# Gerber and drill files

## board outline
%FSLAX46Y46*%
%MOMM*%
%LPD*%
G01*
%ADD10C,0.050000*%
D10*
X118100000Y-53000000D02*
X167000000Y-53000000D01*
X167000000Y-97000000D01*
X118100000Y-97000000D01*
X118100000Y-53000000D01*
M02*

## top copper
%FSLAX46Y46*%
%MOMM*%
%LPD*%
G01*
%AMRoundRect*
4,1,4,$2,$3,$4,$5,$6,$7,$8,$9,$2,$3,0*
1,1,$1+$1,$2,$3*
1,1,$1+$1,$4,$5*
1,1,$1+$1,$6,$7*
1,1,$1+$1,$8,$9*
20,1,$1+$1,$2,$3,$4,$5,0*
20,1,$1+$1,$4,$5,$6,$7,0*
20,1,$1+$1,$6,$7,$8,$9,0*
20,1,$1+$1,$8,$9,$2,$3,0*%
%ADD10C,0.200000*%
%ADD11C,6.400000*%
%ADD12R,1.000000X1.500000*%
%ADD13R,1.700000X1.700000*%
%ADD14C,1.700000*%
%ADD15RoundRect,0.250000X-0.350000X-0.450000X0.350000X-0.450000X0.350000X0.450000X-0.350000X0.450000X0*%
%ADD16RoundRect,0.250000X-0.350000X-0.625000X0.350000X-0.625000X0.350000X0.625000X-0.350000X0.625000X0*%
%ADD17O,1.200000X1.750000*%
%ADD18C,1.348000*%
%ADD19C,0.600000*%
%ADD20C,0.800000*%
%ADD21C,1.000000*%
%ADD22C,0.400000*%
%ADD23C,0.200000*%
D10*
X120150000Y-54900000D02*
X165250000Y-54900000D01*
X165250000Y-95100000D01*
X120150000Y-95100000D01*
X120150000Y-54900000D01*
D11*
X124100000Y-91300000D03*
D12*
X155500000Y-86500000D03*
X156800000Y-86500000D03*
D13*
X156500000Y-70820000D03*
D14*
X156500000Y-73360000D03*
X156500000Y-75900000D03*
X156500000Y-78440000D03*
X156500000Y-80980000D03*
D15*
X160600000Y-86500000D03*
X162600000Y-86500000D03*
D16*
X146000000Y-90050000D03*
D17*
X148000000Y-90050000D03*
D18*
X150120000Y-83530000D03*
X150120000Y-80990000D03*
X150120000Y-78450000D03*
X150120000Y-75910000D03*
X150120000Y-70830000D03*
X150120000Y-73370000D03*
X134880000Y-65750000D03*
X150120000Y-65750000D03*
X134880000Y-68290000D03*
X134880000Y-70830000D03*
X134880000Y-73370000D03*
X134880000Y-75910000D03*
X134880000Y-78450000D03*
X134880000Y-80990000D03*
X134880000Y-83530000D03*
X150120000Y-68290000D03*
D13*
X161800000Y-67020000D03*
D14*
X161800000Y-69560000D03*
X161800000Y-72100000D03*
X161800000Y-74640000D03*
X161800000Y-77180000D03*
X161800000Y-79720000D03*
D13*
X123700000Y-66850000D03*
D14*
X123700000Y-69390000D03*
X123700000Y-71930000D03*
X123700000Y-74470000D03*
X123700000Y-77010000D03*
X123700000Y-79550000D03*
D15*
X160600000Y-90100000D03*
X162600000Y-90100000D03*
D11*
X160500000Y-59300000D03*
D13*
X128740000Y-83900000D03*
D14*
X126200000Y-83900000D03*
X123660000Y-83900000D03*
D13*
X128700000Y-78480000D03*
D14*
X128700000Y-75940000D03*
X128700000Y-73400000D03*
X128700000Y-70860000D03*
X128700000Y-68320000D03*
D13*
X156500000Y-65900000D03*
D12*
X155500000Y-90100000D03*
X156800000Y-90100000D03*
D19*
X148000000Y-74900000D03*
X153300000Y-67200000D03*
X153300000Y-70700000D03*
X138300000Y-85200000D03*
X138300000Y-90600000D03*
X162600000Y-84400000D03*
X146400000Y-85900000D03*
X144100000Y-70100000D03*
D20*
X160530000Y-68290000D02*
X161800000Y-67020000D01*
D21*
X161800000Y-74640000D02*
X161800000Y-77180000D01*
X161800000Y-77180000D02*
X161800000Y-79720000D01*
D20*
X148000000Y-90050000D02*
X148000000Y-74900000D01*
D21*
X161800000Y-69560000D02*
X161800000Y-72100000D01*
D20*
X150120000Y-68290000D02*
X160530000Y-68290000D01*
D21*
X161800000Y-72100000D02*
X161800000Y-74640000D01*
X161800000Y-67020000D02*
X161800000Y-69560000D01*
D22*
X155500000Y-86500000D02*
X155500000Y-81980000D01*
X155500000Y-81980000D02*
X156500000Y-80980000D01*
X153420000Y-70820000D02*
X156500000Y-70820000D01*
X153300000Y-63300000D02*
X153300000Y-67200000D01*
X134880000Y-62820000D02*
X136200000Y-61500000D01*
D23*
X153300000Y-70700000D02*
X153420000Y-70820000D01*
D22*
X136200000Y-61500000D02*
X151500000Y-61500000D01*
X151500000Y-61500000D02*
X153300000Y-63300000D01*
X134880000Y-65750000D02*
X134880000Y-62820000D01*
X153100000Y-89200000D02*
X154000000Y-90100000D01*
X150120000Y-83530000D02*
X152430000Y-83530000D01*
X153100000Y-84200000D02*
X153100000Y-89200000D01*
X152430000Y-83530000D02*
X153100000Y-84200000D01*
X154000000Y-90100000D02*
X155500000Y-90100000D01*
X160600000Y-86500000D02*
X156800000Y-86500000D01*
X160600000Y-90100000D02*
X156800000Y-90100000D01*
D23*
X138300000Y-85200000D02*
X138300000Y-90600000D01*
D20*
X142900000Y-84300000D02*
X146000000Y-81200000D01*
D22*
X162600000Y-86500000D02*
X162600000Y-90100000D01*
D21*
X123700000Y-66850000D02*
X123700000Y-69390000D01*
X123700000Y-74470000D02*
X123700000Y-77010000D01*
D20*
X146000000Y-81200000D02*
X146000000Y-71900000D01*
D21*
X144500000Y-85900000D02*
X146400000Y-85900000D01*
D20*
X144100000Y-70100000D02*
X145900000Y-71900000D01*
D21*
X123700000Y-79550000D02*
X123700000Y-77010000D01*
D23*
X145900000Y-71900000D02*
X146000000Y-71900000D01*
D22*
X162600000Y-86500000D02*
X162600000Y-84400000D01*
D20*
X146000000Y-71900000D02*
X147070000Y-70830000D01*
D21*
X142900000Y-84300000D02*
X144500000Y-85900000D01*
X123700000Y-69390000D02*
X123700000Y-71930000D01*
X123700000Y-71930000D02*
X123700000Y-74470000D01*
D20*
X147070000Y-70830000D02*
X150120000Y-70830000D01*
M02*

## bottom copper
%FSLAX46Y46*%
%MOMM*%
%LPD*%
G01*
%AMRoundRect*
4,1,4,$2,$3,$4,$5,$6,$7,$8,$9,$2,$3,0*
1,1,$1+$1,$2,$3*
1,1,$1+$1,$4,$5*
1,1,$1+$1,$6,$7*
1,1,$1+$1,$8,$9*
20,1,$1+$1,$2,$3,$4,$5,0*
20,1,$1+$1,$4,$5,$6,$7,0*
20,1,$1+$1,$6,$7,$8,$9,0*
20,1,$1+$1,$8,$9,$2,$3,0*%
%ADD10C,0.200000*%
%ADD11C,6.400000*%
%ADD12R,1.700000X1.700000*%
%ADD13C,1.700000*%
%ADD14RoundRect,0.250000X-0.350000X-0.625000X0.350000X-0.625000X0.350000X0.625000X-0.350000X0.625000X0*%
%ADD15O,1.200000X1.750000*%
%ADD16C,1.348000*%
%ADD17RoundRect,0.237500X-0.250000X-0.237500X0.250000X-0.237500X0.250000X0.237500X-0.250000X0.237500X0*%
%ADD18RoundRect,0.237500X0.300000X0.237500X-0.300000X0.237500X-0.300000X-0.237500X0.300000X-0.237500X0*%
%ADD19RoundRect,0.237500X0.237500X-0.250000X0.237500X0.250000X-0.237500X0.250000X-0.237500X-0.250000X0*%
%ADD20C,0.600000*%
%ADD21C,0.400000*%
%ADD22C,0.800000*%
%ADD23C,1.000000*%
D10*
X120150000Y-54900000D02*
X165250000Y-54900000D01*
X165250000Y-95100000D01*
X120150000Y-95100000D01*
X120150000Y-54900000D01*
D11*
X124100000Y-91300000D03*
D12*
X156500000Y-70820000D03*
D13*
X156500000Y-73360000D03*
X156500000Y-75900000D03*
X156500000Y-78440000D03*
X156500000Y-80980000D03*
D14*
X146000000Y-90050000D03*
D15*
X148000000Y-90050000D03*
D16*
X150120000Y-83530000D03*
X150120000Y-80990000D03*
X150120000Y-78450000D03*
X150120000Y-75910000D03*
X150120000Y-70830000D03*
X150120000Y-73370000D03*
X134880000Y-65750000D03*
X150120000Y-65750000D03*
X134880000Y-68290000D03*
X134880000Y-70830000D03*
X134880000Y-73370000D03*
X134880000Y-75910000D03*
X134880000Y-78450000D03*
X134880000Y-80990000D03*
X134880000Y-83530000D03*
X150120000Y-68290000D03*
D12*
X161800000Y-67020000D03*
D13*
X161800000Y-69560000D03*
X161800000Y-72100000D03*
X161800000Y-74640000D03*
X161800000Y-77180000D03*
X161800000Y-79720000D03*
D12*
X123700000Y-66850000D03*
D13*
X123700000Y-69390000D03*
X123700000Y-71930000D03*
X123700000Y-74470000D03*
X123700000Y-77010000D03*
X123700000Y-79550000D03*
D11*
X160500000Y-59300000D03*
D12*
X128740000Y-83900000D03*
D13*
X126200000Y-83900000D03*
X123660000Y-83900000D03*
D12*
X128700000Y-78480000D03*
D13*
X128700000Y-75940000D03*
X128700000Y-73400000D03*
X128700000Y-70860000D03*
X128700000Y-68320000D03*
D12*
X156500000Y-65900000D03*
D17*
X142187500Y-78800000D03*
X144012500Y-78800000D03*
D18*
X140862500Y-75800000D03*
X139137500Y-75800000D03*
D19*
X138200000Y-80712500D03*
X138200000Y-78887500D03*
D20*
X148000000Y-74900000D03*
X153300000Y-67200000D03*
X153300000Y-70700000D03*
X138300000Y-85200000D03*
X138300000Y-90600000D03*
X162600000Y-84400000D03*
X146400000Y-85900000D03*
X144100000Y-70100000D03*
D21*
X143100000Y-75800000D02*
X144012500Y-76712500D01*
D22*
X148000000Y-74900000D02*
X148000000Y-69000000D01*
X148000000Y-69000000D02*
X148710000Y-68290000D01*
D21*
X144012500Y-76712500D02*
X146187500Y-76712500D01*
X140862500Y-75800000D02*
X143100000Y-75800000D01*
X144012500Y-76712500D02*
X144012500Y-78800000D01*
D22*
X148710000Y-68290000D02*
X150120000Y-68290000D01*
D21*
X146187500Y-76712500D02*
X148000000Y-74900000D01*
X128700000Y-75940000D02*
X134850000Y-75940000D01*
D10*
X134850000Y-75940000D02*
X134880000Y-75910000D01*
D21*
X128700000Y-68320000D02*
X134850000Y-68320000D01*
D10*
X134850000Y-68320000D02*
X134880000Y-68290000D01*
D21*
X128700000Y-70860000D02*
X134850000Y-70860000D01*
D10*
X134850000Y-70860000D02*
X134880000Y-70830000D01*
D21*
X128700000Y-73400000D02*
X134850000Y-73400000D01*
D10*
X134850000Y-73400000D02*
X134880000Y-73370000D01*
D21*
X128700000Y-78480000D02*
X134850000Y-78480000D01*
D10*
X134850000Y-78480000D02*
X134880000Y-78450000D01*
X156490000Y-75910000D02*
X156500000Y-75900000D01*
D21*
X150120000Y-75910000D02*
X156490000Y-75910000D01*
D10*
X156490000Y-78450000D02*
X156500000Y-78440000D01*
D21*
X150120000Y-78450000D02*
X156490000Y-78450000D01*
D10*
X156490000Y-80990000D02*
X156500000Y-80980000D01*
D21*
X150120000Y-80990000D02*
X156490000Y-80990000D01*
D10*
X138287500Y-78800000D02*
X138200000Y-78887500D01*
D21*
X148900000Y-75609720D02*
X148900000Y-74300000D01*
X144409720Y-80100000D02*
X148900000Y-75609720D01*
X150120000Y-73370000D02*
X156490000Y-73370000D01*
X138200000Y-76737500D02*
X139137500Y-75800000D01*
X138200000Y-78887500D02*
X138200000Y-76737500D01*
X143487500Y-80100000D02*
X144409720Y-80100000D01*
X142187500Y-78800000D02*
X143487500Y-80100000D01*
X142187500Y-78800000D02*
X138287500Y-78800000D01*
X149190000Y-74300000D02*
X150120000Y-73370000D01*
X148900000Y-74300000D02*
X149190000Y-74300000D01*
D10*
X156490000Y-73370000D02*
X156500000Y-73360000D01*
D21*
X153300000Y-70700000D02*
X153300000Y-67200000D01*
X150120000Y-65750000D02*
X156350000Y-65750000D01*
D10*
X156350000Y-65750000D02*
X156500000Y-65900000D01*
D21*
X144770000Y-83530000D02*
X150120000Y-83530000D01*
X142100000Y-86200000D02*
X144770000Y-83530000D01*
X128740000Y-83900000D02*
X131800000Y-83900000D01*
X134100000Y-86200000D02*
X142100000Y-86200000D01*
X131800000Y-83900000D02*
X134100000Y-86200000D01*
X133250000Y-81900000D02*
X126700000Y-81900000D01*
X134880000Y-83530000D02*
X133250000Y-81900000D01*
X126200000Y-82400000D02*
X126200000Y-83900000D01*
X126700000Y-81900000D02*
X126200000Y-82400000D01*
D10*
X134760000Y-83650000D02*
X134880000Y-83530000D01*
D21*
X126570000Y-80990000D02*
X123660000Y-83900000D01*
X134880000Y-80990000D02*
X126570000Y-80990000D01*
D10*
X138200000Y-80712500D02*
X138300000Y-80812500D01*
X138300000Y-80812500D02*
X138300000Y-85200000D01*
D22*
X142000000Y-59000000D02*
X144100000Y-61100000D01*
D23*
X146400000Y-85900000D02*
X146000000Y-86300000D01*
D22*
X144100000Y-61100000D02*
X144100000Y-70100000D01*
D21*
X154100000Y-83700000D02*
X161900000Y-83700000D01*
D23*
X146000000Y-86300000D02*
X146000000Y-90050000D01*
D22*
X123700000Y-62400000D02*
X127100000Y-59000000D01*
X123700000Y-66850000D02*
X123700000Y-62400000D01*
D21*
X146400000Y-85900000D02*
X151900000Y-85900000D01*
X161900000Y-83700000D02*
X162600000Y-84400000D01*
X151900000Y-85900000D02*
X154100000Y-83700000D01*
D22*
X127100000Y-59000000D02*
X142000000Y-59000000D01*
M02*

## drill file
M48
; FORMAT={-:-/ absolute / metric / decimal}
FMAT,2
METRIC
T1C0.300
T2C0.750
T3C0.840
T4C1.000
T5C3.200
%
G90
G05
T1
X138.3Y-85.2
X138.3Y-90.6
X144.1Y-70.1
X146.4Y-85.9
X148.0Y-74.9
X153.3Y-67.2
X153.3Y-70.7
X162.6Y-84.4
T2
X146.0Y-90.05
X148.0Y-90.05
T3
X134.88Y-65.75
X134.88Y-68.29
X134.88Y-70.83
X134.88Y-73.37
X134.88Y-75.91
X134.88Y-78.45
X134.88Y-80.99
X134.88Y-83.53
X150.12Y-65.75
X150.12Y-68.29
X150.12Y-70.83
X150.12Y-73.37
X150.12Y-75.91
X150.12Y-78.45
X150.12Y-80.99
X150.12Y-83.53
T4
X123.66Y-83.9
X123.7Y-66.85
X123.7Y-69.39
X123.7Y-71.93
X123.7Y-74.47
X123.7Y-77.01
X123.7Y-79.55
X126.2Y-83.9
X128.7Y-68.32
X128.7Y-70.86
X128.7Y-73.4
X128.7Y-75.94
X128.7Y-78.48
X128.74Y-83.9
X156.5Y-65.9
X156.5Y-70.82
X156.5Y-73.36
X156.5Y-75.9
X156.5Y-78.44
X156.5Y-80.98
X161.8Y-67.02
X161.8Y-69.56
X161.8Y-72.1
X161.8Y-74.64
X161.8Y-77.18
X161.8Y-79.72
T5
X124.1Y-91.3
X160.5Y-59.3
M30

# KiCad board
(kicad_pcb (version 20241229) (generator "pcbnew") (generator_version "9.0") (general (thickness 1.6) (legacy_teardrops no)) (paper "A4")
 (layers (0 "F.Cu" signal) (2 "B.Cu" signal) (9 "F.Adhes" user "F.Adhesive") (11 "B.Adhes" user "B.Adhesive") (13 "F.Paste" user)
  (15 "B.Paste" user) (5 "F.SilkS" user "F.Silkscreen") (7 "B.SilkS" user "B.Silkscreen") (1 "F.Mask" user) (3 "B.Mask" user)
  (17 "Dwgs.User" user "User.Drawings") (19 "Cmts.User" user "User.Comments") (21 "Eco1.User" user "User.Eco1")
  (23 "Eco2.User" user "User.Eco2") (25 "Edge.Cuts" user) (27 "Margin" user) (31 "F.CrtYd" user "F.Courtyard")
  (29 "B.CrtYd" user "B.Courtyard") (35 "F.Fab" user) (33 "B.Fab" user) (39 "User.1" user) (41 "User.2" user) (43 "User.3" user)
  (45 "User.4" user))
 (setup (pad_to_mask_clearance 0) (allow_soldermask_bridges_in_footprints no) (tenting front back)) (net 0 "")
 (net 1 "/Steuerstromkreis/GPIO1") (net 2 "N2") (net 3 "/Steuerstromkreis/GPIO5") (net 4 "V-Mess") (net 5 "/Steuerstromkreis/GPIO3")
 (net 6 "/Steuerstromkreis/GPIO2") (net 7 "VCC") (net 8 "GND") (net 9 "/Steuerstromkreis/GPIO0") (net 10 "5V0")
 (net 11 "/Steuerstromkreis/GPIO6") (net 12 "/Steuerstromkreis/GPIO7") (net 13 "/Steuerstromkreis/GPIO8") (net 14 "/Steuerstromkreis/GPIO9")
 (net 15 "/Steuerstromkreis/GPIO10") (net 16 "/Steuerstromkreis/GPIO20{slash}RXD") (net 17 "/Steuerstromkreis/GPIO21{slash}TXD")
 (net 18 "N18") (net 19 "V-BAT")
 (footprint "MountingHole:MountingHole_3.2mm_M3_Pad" (layer "F.Cu") (at 124.1 91.3)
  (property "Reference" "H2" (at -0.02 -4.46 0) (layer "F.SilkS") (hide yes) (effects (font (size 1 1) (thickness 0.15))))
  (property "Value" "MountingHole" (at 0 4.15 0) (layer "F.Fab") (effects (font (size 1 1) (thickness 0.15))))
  (pad "1" thru_hole circle (at 0 0) (size 6.4 6.4) (drill 3.2) (layers "*.Cu" "*.Mask") (remove_unused_layers no) (zone_connect 2)))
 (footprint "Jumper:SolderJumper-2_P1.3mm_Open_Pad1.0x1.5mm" (layer "F.Cu") (at 156.15 86.5)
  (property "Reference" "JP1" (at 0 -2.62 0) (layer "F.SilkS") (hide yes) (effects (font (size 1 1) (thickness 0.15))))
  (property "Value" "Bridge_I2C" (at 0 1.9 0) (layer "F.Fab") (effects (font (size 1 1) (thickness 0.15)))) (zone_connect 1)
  (pad "1" smd rect (at -0.65 0) (size 1 1.5) (layers "F.Cu" "F.Mask") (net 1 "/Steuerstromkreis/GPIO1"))
  (pad "2" smd rect (at 0.65 0) (size 1 1.5) (layers "F.Cu" "F.Mask") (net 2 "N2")))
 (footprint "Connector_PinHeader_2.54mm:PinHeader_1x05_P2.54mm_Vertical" (layer "F.Cu") (at 156.5 70.82)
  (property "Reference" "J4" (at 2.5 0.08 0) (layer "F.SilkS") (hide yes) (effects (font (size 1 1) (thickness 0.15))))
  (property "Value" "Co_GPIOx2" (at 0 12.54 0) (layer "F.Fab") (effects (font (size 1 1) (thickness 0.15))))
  (pad "1" thru_hole rect (at 0 0) (size 1.7 1.7) (drill 1) (layers "*.Cu" "*.Mask") (remove_unused_layers no)
   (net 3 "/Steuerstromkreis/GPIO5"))
  (pad "2" thru_hole circle (at 0 2.54) (size 1.7 1.7) (drill 1) (layers "*.Cu" "*.Mask") (remove_unused_layers no) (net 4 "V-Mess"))
  (pad "3" thru_hole circle (at 0 5.08) (size 1.7 1.7) (drill 1) (layers "*.Cu" "*.Mask") (remove_unused_layers no)
   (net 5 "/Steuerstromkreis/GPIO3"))
  (pad "4" thru_hole circle (at 0 7.62) (size 1.7 1.7) (drill 1) (layers "*.Cu" "*.Mask") (remove_unused_layers no)
   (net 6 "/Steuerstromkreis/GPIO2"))
  (pad "5" thru_hole circle (at 0 10.16) (size 1.7 1.7) (drill 1) (layers "*.Cu" "*.Mask") (remove_unused_layers no)
   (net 1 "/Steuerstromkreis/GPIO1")))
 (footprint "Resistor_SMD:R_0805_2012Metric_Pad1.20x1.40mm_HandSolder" (layer "F.Cu") (at 161.6 86.5)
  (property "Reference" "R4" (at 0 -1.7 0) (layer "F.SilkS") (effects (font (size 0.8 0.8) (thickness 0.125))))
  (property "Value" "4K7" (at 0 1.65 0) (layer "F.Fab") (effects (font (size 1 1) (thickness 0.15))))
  (pad "1" smd roundrect (at -1 0) (size 1.2 1.4) (layers "F.Cu" "F.Mask" "F.Paste") (roundrect_rratio 0.208333) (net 2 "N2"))
  (pad "2" smd roundrect (at 1 0) (size 1.2 1.4) (layers "F.Cu" "F.Mask" "F.Paste") (roundrect_rratio 0.208333) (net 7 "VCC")))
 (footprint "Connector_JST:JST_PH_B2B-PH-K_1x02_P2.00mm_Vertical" (layer "F.Cu") (at 146 90.05)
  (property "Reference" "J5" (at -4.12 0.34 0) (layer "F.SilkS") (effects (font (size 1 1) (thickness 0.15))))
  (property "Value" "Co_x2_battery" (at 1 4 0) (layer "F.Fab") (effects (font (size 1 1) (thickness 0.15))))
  (pad "1" thru_hole roundrect (at 0 0) (size 1.2 1.75) (drill 0.75) (layers "*.Cu" "*.Mask") (remove_unused_layers no)
   (roundrect_rratio 0.208333) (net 7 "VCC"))
  (pad "2" thru_hole oval (at 2 0) (size 1.2 1.75) (drill 0.75) (layers "*.Cu" "*.Mask") (remove_unused_layers no) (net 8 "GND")))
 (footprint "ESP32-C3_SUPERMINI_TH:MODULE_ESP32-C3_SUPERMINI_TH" (layer "F.Cu") (at 142.5 75.65)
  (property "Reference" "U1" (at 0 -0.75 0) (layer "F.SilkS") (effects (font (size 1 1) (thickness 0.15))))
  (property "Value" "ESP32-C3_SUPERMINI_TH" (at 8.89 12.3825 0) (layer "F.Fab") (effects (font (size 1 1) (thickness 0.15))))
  (pad "0" thru_hole circle (at 7.62 7.88) (size 1.348 1.348) (drill 0.84) (layers "*.Cu" "*.Mask") (remove_unused_layers no)
   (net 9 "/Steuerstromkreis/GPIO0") (solder_mask_margin 0.102))
  (pad "1" thru_hole circle (at 7.62 5.34) (size 1.348 1.348) (drill 0.84) (layers "*.Cu" "*.Mask") (remove_unused_layers no)
   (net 1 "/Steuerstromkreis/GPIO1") (solder_mask_margin 0.102))
  (pad "2" thru_hole circle (at 7.62 2.8) (size 1.348 1.348) (drill 0.84) (layers "*.Cu" "*.Mask") (remove_unused_layers no)
   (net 6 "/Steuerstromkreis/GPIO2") (solder_mask_margin 0.102))
  (pad "3" thru_hole circle (at 7.62 0.26) (size 1.348 1.348) (drill 0.84) (layers "*.Cu" "*.Mask") (remove_unused_layers no)
   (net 5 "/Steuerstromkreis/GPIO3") (solder_mask_margin 0.102))
  (pad "3.3" thru_hole circle (at 7.62 -4.82) (size 1.348 1.348) (drill 0.84) (layers "*.Cu" "*.Mask") (remove_unused_layers no)
   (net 7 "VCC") (solder_mask_margin 0.102))
  (pad "4" thru_hole circle (at 7.62 -2.28) (size 1.348 1.348) (drill 0.84) (layers "*.Cu" "*.Mask") (remove_unused_layers no)
   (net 4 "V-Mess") (solder_mask_margin 0.102))
  (pad "5" thru_hole circle (at -7.62 -9.9) (size 1.348 1.348) (drill 0.84) (layers "*.Cu" "*.Mask") (remove_unused_layers no)
   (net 3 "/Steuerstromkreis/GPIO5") (solder_mask_margin 0.102))
  (pad "5V" thru_hole circle (at 7.62 -9.9) (size 1.348 1.348) (drill 0.84) (layers "*.Cu" "*.Mask") (remove_unused_layers no)
   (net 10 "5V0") (solder_mask_margin 0.102))
  (pad "6" thru_hole circle (at -7.62 -7.36) (size 1.348 1.348) (drill 0.84) (layers "*.Cu" "*.Mask") (remove_unused_layers no)
   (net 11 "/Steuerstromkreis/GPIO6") (solder_mask_margin 0.102))
  (pad "7" thru_hole circle (at -7.62 -4.82) (size 1.348 1.348) (drill 0.84) (layers "*.Cu" "*.Mask") (remove_unused_layers no)
   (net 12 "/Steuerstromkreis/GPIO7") (solder_mask_margin 0.102))
  (pad "8" thru_hole circle (at -7.62 -2.28) (size 1.348 1.348) (drill 0.84) (layers "*.Cu" "*.Mask") (remove_unused_layers no)
   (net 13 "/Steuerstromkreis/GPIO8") (solder_mask_margin 0.102))
  (pad "9" thru_hole circle (at -7.62 0.26) (size 1.348 1.348) (drill 0.84) (layers "*.Cu" "*.Mask") (remove_unused_layers no)
   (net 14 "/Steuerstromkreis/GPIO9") (solder_mask_margin 0.102))
  (pad "10" thru_hole circle (at -7.62 2.8) (size 1.348 1.348) (drill 0.84) (layers "*.Cu" "*.Mask") (remove_unused_layers no)
   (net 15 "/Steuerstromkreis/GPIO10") (solder_mask_margin 0.102))
  (pad "20" thru_hole circle (at -7.62 5.34) (size 1.348 1.348) (drill 0.84) (layers "*.Cu" "*.Mask") (remove_unused_layers no)
   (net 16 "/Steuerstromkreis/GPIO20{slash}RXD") (solder_mask_margin 0.102))
  (pad "21" thru_hole circle (at -7.62 7.88) (size 1.348 1.348) (drill 0.84) (layers "*.Cu" "*.Mask") (remove_unused_layers no)
   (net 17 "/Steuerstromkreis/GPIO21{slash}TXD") (solder_mask_margin 0.102))
  (pad "G" thru_hole circle (at 7.62 -7.36) (size 1.348 1.348) (drill 0.84) (layers "*.Cu" "*.Mask") (remove_unused_layers no) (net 8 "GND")
   (solder_mask_margin 0.102)))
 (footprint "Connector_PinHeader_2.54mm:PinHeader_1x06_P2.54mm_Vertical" (layer "F.Cu") (at 161.8 67.02)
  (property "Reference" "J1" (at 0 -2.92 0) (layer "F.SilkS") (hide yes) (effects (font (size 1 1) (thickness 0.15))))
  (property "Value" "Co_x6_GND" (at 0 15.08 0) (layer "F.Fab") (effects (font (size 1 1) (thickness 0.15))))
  (pad "1" thru_hole rect (at 0 0) (size 1.7 1.7) (drill 1) (layers "*.Cu" "*.Mask") (remove_unused_layers no) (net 8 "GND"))
  (pad "2" thru_hole circle (at 0 2.54) (size 1.7 1.7) (drill 1) (layers "*.Cu" "*.Mask") (remove_unused_layers no) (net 8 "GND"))
  (pad "3" thru_hole circle (at 0 5.08) (size 1.7 1.7) (drill 1) (layers "*.Cu" "*.Mask") (remove_unused_layers no) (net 8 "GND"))
  (pad "4" thru_hole circle (at 0 7.62) (size 1.7 1.7) (drill 1) (layers "*.Cu" "*.Mask") (remove_unused_layers no) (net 8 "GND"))
  (pad "5" thru_hole circle (at 0 10.16) (size 1.7 1.7) (drill 1) (layers "*.Cu" "*.Mask") (remove_unused_layers no) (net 8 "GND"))
  (pad "6" thru_hole circle (at 0 12.7) (size 1.7 1.7) (drill 1) (layers "*.Cu" "*.Mask") (remove_unused_layers no) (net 8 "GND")))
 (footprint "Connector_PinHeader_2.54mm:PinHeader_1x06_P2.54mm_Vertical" (layer "F.Cu") (at 123.7 66.85)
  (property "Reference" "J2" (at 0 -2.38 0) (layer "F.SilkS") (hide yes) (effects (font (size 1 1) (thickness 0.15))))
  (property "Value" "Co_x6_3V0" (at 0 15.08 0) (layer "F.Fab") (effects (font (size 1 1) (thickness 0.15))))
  (pad "1" thru_hole rect (at 0 0) (size 1.7 1.7) (drill 1) (layers "*.Cu" "*.Mask") (remove_unused_layers no) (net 7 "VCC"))
  (pad "2" thru_hole circle (at 0 2.54) (size 1.7 1.7) (drill 1) (layers "*.Cu" "*.Mask") (remove_unused_layers no) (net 7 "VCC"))
  (pad "3" thru_hole circle (at 0 5.08) (size 1.7 1.7) (drill 1) (layers "*.Cu" "*.Mask") (remove_unused_layers no) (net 7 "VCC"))
  (pad "4" thru_hole circle (at 0 7.62) (size 1.7 1.7) (drill 1) (layers "*.Cu" "*.Mask") (remove_unused_layers no) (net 7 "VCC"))
  (pad "5" thru_hole circle (at 0 10.16) (size 1.7 1.7) (drill 1) (layers "*.Cu" "*.Mask") (remove_unused_layers no) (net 7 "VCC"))
  (pad "6" thru_hole circle (at 0 12.7) (size 1.7 1.7) (drill 1) (layers "*.Cu" "*.Mask") (remove_unused_layers no) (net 7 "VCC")))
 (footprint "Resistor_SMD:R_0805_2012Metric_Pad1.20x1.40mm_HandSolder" (layer "F.Cu") (at 161.6 90.1)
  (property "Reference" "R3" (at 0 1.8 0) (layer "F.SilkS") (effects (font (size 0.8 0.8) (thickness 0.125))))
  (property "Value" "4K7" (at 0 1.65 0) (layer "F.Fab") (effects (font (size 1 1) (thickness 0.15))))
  (pad "1" smd roundrect (at -1 0) (size 1.2 1.4) (layers "F.Cu" "F.Mask" "F.Paste") (roundrect_rratio 0.208333) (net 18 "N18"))
  (pad "2" smd roundrect (at 1 0) (size 1.2 1.4) (layers "F.Cu" "F.Mask" "F.Paste") (roundrect_rratio 0.208333) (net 7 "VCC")))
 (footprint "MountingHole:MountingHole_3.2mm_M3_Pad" (layer "F.Cu") (at 160.5 59.3)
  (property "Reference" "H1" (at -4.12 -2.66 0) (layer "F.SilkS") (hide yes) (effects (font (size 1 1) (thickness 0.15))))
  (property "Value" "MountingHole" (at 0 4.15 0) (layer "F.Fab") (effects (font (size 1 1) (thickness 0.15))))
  (pad "1" thru_hole circle (at 0 0) (size 6.4 6.4) (drill 3.2) (layers "*.Cu" "*.Mask") (remove_unused_layers no) (zone_connect 2)))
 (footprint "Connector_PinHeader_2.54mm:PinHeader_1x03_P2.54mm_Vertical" (layer "F.Cu") (at 128.74 83.9 -90)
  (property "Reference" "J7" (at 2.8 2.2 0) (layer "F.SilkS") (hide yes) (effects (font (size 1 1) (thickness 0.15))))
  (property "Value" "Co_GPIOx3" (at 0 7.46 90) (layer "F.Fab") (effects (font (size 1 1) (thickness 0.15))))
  (pad "1" thru_hole rect (at 0 0 270) (size 1.7 1.7) (drill 1) (layers "*.Cu" "*.Mask") (remove_unused_layers no)
   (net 9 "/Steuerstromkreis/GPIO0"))
  (pad "2" thru_hole circle (at 0 2.54 270) (size 1.7 1.7) (drill 1) (layers "*.Cu" "*.Mask") (remove_unused_layers no)
   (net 17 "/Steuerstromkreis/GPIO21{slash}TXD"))
  (pad "3" thru_hole circle (at 0 5.08 270) (size 1.7 1.7) (drill 1) (layers "*.Cu" "*.Mask") (remove_unused_layers no)
   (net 16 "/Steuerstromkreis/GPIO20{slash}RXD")))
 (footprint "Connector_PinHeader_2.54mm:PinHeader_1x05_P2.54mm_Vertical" (layer "F.Cu") (at 128.7 78.48 180)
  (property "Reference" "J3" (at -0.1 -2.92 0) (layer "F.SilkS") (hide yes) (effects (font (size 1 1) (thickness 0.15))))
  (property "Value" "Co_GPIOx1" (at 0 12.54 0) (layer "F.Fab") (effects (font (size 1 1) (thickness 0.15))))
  (pad "1" thru_hole rect (at 0 0 180) (size 1.7 1.7) (drill 1) (layers "*.Cu" "*.Mask") (remove_unused_layers no)
   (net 15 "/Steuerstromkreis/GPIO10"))
  (pad "2" thru_hole circle (at 0 2.54 180) (size 1.7 1.7) (drill 1) (layers "*.Cu" "*.Mask") (remove_unused_layers no)
   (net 14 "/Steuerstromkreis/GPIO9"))
  (pad "3" thru_hole circle (at 0 5.08 180) (size 1.7 1.7) (drill 1) (layers "*.Cu" "*.Mask") (remove_unused_layers no)
   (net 13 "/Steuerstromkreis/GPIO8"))
  (pad "4" thru_hole circle (at 0 7.62 180) (size 1.7 1.7) (drill 1) (layers "*.Cu" "*.Mask") (remove_unused_layers no)
   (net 12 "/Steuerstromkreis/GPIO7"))
  (pad "5" thru_hole circle (at 0 10.16 180) (size 1.7 1.7) (drill 1) (layers "*.Cu" "*.Mask") (remove_unused_layers no)
   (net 11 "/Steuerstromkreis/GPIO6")))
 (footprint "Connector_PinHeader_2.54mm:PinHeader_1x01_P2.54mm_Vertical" (layer "F.Cu") (at 156.5 65.9)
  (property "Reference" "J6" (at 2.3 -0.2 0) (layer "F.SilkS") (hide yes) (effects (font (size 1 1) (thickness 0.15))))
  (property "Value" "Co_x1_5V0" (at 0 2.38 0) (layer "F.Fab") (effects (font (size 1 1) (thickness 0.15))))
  (pad "1" thru_hole rect (at 0 0) (size 1.7 1.7) (drill 1) (layers "*.Cu" "*.Mask") (remove_unused_layers no) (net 10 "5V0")))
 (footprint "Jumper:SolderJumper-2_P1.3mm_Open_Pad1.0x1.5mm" (layer "F.Cu") (at 156.15 90.1)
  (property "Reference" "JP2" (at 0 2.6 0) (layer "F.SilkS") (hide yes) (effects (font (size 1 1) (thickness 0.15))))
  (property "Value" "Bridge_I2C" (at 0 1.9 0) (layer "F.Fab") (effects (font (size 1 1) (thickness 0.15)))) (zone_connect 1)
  (pad "1" smd rect (at -0.65 0) (size 1 1.5) (layers "F.Cu" "F.Mask") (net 9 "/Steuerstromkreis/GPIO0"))
  (pad "2" smd rect (at 0.65 0) (size 1 1.5) (layers "F.Cu" "F.Mask") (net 18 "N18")))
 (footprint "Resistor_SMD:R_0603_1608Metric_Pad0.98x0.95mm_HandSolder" (layer "B.Cu") (at 143.1 78.8)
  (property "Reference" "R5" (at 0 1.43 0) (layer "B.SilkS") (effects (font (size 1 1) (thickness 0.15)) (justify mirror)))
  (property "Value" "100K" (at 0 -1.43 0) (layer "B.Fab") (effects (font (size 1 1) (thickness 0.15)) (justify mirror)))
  (pad "1" smd roundrect (at -0.9125 0) (size 0.975 0.95) (layers "B.Cu" "B.Mask" "B.Paste") (roundrect_rratio 0.25) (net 4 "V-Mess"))
  (pad "2" smd roundrect (at 0.9125 0) (size 0.975 0.95) (layers "B.Cu" "B.Mask" "B.Paste") (roundrect_rratio 0.25) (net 8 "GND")))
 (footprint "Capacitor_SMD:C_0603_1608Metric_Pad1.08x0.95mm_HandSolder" (layer "B.Cu") (at 140 75.8 180)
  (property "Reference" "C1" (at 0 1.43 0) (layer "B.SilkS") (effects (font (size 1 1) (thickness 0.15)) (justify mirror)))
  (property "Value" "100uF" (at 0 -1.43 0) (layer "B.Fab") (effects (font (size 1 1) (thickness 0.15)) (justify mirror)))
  (pad "1" smd roundrect (at -0.8625 0 180) (size 1.075 0.95) (layers "B.Cu" "B.Mask" "B.Paste") (roundrect_rratio 0.25) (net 8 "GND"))
  (pad "2" smd roundrect (at 0.8625 0 180) (size 1.075 0.95) (layers "B.Cu" "B.Mask" "B.Paste") (roundrect_rratio 0.25) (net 4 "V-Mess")))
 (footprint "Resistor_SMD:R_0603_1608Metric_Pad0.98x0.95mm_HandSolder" (layer "B.Cu") (at 138.2 79.8 90)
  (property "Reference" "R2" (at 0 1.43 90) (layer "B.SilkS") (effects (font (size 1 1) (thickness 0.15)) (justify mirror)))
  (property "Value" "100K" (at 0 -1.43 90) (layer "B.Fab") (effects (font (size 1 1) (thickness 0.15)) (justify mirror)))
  (pad "1" smd roundrect (at -0.9125 0 90) (size 0.975 0.95) (layers "B.Cu" "B.Mask" "B.Paste") (roundrect_rratio 0.25) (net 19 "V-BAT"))
  (pad "2" smd roundrect (at 0.9125 0 90) (size 0.975 0.95) (layers "B.Cu" "B.Mask" "B.Paste") (roundrect_rratio 0.25) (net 4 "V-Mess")))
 (gr_rect (start 120.15 54.9) (end 165.25 95.1) (stroke (width 0.2) (type default)) (fill no) (layer "F.Cu"))
 (gr_rect (start 120.15 54.9) (end 165.25 95.1) (stroke (width 0.2) (type default)) (fill no) (layer "B.Cu") (net 16))
 (gr_rect (start 118.1 53) (end 167 97) (stroke (width 0.05) (type default)) (fill no) (layer "Edge.Cuts"))
 (segment (start 160.53 68.29) (end 161.8 67.02) (width 0.8) (layer "F.Cu") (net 8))
 (segment (start 161.8 74.64) (end 161.8 77.18) (width 1) (layer "F.Cu") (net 8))
 (segment (start 161.8 77.18) (end 161.8 79.72) (width 1) (layer "F.Cu") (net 8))
 (segment (start 148 90.05) (end 148 74.9) (width 0.8) (layer "F.Cu") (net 8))
 (segment (start 161.8 69.56) (end 161.8 72.1) (width 1) (layer "F.Cu") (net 8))
 (segment (start 150.12 68.29) (end 160.53 68.29) (width 0.8) (layer "F.Cu") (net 8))
 (segment (start 161.8 72.1) (end 161.8 74.64) (width 1) (layer "F.Cu") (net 8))
 (segment (start 161.8 67.02) (end 161.8 69.56) (width 1) (layer "F.Cu") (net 8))
 (via (at 148 74.9) (size 0.6) (drill 0.3) (layers "F.Cu" "B.Cu") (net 8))
 (segment (start 143.1 75.8) (end 144.0125 76.7125) (width 0.4) (layer "B.Cu") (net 8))
 (segment (start 148 74.9) (end 148 69) (width 0.8) (layer "B.Cu") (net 8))
 (segment (start 148 69) (end 148.71 68.29) (width 0.8) (layer "B.Cu") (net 8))
 (segment (start 144.0125 76.7125) (end 146.1875 76.7125) (width 0.4) (layer "B.Cu") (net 8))
 (segment (start 140.8625 75.8) (end 143.1 75.8) (width 0.4) (layer "B.Cu") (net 8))
 (segment (start 144.0125 76.7125) (end 144.0125 78.8) (width 0.4) (layer "B.Cu") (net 8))
 (segment (start 148.71 68.29) (end 150.12 68.29) (width 0.8) (layer "B.Cu") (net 8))
 (segment (start 146.1875 76.7125) (end 148 74.9) (width 0.4) (layer "B.Cu") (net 8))
 (segment (start 128.7 75.94) (end 134.85 75.94) (width 0.4) (layer "B.Cu") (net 14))
 (segment (start 134.85 75.94) (end 134.88 75.91) (width 0.2) (layer "B.Cu") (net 14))
 (segment (start 128.7 68.32) (end 134.85 68.32) (width 0.4) (layer "B.Cu") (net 11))
 (segment (start 134.85 68.32) (end 134.88 68.29) (width 0.2) (layer "B.Cu") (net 11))
 (segment (start 128.7 70.86) (end 134.85 70.86) (width 0.4) (layer "B.Cu") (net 12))
 (segment (start 134.85 70.86) (end 134.88 70.83) (width 0.2) (layer "B.Cu") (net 12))
 (segment (start 128.7 73.4) (end 134.85 73.4) (width 0.4) (layer "B.Cu") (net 13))
 (segment (start 134.85 73.4) (end 134.88 73.37) (width 0.2) (layer "B.Cu") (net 13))
 (segment (start 128.7 78.48) (end 134.85 78.48) (width 0.4) (layer "B.Cu") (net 15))
 (segment (start 134.85 78.48) (end 134.88 78.45) (width 0.2) (layer "B.Cu") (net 15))
 (segment (start 156.49 75.91) (end 156.5 75.9) (width 0.2) (layer "B.Cu") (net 5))
 (segment (start 150.12 75.91) (end 156.49 75.91) (width 0.4) (layer "B.Cu") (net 5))
 (segment (start 156.49 78.45) (end 156.5 78.44) (width 0.2) (layer "B.Cu") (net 6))
 (segment (start 150.12 78.45) (end 156.49 78.45) (width 0.4) (layer "B.Cu") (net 6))
 (segment (start 155.5 86.5) (end 155.5 81.98) (width 0.4) (layer "F.Cu") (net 1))
 (segment (start 155.5 81.98) (end 156.5 80.98) (width 0.4) (layer "F.Cu") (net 1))
 (segment (start 156.49 80.99) (end 156.5 80.98) (width 0.2) (layer "B.Cu") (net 1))
 (segment (start 150.12 80.99) (end 156.49 80.99) (width 0.4) (layer "B.Cu") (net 1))
 (segment (start 138.2875 78.8) (end 138.2 78.8875) (width 0.2) (layer "B.Cu") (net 4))
 (segment (start 148.9 75.60972) (end 148.9 74.3) (width 0.4) (layer "B.Cu") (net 4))
 (segment (start 144.40972 80.1) (end 148.9 75.60972) (width 0.4) (layer "B.Cu") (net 4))
 (segment (start 150.12 73.37) (end 156.49 73.37) (width 0.4) (layer "B.Cu") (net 4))
 (segment (start 138.2 76.7375) (end 139.1375 75.8) (width 0.4) (layer "B.Cu") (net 4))
 (segment (start 138.2 78.8875) (end 138.2 76.7375) (width 0.4) (layer "B.Cu") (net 4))
 (segment (start 143.4875 80.1) (end 144.40972 80.1) (width 0.4) (layer "B.Cu") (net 4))
 (segment (start 142.1875 78.8) (end 143.4875 80.1) (width 0.4) (layer "B.Cu") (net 4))
 (segment (start 142.1875 78.8) (end 138.2875 78.8) (width 0.4) (layer "B.Cu") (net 4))
 (segment (start 149.19 74.3) (end 150.12 73.37) (width 0.4) (layer "B.Cu") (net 4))
 (segment (start 148.9 74.3) (end 149.19 74.3) (width 0.4) (layer "B.Cu") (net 4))
 (segment (start 156.49 73.37) (end 156.5 73.36) (width 0.2) (layer "B.Cu") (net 4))
 (segment (start 153.42 70.82) (end 156.5 70.82) (width 0.4) (layer "F.Cu") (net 3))
 (segment (start 153.3 63.3) (end 153.3 67.2) (width 0.4) (layer "F.Cu") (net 3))
 (segment (start 134.88 62.82) (end 136.2 61.5) (width 0.4) (layer "F.Cu") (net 3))
 (segment (start 153.3 70.7) (end 153.42 70.82) (width 0.2) (layer "F.Cu") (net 3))
 (segment (start 136.2 61.5) (end 151.5 61.5) (width 0.4) (layer "F.Cu") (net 3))
 (segment (start 151.5 61.5) (end 153.3 63.3) (width 0.4) (layer "F.Cu") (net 3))
 (segment (start 134.88 65.75) (end 134.88 62.82) (width 0.4) (layer "F.Cu") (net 3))
 (via (at 153.3 67.2) (size 0.6) (drill 0.3) (layers "F.Cu" "B.Cu") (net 3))
 (via (at 153.3 70.7) (size 0.6) (drill 0.3) (layers "F.Cu" "B.Cu") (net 3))
 (segment (start 153.3 70.7) (end 153.3 67.2) (width 0.4) (layer "B.Cu") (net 3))
 (segment (start 150.12 65.75) (end 156.35 65.75) (width 0.4) (layer "B.Cu") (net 10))
 (segment (start 156.35 65.75) (end 156.5 65.9) (width 0.2) (layer "B.Cu") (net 10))
 (segment (start 153.1 89.2) (end 154 90.1) (width 0.4) (layer "F.Cu") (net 9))
 (segment (start 150.12 83.53) (end 152.43 83.53) (width 0.4) (layer "F.Cu") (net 9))
 (segment (start 153.1 84.2) (end 153.1 89.2) (width 0.4) (layer "F.Cu") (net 9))
 (segment (start 152.43 83.53) (end 153.1 84.2) (width 0.4) (layer "F.Cu") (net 9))
 (segment (start 154 90.1) (end 155.5 90.1) (width 0.4) (layer "F.Cu") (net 9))
 (segment (start 144.77 83.53) (end 150.12 83.53) (width 0.4) (layer "B.Cu") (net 9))
 (segment (start 142.1 86.2) (end 144.77 83.53) (width 0.4) (layer "B.Cu") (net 9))
 (segment (start 128.74 83.9) (end 131.8 83.9) (width 0.4) (layer "B.Cu") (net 9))
 (segment (start 134.1 86.2) (end 142.1 86.2) (width 0.4) (layer "B.Cu") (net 9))
 (segment (start 131.8 83.9) (end 134.1 86.2) (width 0.4) (layer "B.Cu") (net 9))
 (segment (start 133.25 81.9) (end 126.7 81.9) (width 0.4) (layer "B.Cu") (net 17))
 (segment (start 134.88 83.53) (end 133.25 81.9) (width 0.4) (layer "B.Cu") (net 17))
 (segment (start 126.2 82.4) (end 126.2 83.9) (width 0.4) (layer "B.Cu") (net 17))
 (segment (start 126.7 81.9) (end 126.2 82.4) (width 0.4) (layer "B.Cu") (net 17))
 (segment (start 134.76 83.65) (end 134.88 83.53) (width 0.2) (layer "B.Cu") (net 17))
 (segment (start 126.57 80.99) (end 123.66 83.9) (width 0.4) (layer "B.Cu") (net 16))
 (segment (start 134.88 80.99) (end 126.57 80.99) (width 0.4) (layer "B.Cu") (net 16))
 (segment (start 160.6 86.5) (end 156.8 86.5) (width 0.4) (layer "F.Cu") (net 2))
 (segment (start 160.6 90.1) (end 156.8 90.1) (width 0.4) (layer "F.Cu") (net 18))
 (segment (start 138.3 85.2) (end 138.3 90.6) (width 0.2) (layer "F.Cu") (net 19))
 (via (at 138.3 85.2) (size 0.6) (drill 0.3) (layers "F.Cu" "B.Cu") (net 19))
 (via (at 138.3 90.6) (size 0.6) (drill 0.3) (layers "F.Cu" "B.Cu") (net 19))
 (segment (start 138.2 80.7125) (end 138.3 80.8125) (width 0.2) (layer "B.Cu") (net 19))
 (segment (start 138.3 80.8125) (end 138.3 85.2) (width 0.2) (layer "B.Cu") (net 19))
 (segment (start 142.9 84.3) (end 146 81.2) (width 0.8) (layer "F.Cu") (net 7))
 (segment (start 162.6 86.5) (end 162.6 90.1) (width 0.4) (layer "F.Cu") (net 7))
 (segment (start 123.7 66.85) (end 123.7 69.39) (width 1) (layer "F.Cu") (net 7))
 (segment (start 123.7 74.47) (end 123.7 77.01) (width 1) (layer "F.Cu") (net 7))
 (segment (start 146 81.2) (end 146 71.9) (width 0.8) (layer "F.Cu") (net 7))
 (segment (start 144.5 85.9) (end 146.4 85.9) (width 1) (layer "F.Cu") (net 7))
 (segment (start 144.1 70.1) (end 145.9 71.9) (width 0.8) (layer "F.Cu") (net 7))
 (segment (start 123.7 79.55) (end 123.7 77.01) (width 1) (layer "F.Cu") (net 7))
 (segment (start 145.9 71.9) (end 146 71.9) (width 0.2) (layer "F.Cu") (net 7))
 (segment (start 162.6 86.5) (end 162.6 84.4) (width 0.4) (layer "F.Cu") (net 7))
 (segment (start 146 71.9) (end 147.07 70.83) (width 0.8) (layer "F.Cu") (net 7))
 (segment (start 142.9 84.3) (end 144.5 85.9) (width 1) (layer "F.Cu") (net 7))
 (segment (start 123.7 69.39) (end 123.7 71.93) (width 1) (layer "F.Cu") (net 7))
 (segment (start 123.7 71.93) (end 123.7 74.47) (width 1) (layer "F.Cu") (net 7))
 (segment (start 147.07 70.83) (end 150.12 70.83) (width 0.8) (layer "F.Cu") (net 7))
 (via (at 162.6 84.4) (size 0.6) (drill 0.3) (layers "F.Cu" "B.Cu") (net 7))
 (via (at 146.4 85.9) (size 0.6) (drill 0.3) (layers "F.Cu" "B.Cu") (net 7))
 (via (at 144.1 70.1) (size 0.6) (drill 0.3) (layers "F.Cu" "B.Cu") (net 7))
 (segment (start 142 59) (end 144.1 61.1) (width 0.8) (layer "B.Cu") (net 7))
 (segment (start 146.4 85.9) (end 146 86.3) (width 1) (layer "B.Cu") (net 7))
 (segment (start 144.1 61.1) (end 144.1 70.1) (width 0.8) (layer "B.Cu") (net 7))
 (segment (start 154.1 83.7) (end 161.9 83.7) (width 0.4) (layer "B.Cu") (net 7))
 (segment (start 146 86.3) (end 146 90.05) (width 1) (layer "B.Cu") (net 7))
 (segment (start 123.7 62.4) (end 127.1 59) (width 0.8) (layer "B.Cu") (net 7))
 (segment (start 123.7 66.85) (end 123.7 62.4) (width 0.8) (layer "B.Cu") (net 7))
 (segment (start 146.4 85.9) (end 151.9 85.9) (width 0.4) (layer "B.Cu") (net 7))
 (segment (start 161.9 83.7) (end 162.6 84.4) (width 0.4) (layer "B.Cu") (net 7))
 (segment (start 151.9 85.9) (end 154.1 83.7) (width 0.4) (layer "B.Cu") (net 7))
 (segment (start 127.1 59) (end 142 59) (width 0.8) (layer "B.Cu") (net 7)))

